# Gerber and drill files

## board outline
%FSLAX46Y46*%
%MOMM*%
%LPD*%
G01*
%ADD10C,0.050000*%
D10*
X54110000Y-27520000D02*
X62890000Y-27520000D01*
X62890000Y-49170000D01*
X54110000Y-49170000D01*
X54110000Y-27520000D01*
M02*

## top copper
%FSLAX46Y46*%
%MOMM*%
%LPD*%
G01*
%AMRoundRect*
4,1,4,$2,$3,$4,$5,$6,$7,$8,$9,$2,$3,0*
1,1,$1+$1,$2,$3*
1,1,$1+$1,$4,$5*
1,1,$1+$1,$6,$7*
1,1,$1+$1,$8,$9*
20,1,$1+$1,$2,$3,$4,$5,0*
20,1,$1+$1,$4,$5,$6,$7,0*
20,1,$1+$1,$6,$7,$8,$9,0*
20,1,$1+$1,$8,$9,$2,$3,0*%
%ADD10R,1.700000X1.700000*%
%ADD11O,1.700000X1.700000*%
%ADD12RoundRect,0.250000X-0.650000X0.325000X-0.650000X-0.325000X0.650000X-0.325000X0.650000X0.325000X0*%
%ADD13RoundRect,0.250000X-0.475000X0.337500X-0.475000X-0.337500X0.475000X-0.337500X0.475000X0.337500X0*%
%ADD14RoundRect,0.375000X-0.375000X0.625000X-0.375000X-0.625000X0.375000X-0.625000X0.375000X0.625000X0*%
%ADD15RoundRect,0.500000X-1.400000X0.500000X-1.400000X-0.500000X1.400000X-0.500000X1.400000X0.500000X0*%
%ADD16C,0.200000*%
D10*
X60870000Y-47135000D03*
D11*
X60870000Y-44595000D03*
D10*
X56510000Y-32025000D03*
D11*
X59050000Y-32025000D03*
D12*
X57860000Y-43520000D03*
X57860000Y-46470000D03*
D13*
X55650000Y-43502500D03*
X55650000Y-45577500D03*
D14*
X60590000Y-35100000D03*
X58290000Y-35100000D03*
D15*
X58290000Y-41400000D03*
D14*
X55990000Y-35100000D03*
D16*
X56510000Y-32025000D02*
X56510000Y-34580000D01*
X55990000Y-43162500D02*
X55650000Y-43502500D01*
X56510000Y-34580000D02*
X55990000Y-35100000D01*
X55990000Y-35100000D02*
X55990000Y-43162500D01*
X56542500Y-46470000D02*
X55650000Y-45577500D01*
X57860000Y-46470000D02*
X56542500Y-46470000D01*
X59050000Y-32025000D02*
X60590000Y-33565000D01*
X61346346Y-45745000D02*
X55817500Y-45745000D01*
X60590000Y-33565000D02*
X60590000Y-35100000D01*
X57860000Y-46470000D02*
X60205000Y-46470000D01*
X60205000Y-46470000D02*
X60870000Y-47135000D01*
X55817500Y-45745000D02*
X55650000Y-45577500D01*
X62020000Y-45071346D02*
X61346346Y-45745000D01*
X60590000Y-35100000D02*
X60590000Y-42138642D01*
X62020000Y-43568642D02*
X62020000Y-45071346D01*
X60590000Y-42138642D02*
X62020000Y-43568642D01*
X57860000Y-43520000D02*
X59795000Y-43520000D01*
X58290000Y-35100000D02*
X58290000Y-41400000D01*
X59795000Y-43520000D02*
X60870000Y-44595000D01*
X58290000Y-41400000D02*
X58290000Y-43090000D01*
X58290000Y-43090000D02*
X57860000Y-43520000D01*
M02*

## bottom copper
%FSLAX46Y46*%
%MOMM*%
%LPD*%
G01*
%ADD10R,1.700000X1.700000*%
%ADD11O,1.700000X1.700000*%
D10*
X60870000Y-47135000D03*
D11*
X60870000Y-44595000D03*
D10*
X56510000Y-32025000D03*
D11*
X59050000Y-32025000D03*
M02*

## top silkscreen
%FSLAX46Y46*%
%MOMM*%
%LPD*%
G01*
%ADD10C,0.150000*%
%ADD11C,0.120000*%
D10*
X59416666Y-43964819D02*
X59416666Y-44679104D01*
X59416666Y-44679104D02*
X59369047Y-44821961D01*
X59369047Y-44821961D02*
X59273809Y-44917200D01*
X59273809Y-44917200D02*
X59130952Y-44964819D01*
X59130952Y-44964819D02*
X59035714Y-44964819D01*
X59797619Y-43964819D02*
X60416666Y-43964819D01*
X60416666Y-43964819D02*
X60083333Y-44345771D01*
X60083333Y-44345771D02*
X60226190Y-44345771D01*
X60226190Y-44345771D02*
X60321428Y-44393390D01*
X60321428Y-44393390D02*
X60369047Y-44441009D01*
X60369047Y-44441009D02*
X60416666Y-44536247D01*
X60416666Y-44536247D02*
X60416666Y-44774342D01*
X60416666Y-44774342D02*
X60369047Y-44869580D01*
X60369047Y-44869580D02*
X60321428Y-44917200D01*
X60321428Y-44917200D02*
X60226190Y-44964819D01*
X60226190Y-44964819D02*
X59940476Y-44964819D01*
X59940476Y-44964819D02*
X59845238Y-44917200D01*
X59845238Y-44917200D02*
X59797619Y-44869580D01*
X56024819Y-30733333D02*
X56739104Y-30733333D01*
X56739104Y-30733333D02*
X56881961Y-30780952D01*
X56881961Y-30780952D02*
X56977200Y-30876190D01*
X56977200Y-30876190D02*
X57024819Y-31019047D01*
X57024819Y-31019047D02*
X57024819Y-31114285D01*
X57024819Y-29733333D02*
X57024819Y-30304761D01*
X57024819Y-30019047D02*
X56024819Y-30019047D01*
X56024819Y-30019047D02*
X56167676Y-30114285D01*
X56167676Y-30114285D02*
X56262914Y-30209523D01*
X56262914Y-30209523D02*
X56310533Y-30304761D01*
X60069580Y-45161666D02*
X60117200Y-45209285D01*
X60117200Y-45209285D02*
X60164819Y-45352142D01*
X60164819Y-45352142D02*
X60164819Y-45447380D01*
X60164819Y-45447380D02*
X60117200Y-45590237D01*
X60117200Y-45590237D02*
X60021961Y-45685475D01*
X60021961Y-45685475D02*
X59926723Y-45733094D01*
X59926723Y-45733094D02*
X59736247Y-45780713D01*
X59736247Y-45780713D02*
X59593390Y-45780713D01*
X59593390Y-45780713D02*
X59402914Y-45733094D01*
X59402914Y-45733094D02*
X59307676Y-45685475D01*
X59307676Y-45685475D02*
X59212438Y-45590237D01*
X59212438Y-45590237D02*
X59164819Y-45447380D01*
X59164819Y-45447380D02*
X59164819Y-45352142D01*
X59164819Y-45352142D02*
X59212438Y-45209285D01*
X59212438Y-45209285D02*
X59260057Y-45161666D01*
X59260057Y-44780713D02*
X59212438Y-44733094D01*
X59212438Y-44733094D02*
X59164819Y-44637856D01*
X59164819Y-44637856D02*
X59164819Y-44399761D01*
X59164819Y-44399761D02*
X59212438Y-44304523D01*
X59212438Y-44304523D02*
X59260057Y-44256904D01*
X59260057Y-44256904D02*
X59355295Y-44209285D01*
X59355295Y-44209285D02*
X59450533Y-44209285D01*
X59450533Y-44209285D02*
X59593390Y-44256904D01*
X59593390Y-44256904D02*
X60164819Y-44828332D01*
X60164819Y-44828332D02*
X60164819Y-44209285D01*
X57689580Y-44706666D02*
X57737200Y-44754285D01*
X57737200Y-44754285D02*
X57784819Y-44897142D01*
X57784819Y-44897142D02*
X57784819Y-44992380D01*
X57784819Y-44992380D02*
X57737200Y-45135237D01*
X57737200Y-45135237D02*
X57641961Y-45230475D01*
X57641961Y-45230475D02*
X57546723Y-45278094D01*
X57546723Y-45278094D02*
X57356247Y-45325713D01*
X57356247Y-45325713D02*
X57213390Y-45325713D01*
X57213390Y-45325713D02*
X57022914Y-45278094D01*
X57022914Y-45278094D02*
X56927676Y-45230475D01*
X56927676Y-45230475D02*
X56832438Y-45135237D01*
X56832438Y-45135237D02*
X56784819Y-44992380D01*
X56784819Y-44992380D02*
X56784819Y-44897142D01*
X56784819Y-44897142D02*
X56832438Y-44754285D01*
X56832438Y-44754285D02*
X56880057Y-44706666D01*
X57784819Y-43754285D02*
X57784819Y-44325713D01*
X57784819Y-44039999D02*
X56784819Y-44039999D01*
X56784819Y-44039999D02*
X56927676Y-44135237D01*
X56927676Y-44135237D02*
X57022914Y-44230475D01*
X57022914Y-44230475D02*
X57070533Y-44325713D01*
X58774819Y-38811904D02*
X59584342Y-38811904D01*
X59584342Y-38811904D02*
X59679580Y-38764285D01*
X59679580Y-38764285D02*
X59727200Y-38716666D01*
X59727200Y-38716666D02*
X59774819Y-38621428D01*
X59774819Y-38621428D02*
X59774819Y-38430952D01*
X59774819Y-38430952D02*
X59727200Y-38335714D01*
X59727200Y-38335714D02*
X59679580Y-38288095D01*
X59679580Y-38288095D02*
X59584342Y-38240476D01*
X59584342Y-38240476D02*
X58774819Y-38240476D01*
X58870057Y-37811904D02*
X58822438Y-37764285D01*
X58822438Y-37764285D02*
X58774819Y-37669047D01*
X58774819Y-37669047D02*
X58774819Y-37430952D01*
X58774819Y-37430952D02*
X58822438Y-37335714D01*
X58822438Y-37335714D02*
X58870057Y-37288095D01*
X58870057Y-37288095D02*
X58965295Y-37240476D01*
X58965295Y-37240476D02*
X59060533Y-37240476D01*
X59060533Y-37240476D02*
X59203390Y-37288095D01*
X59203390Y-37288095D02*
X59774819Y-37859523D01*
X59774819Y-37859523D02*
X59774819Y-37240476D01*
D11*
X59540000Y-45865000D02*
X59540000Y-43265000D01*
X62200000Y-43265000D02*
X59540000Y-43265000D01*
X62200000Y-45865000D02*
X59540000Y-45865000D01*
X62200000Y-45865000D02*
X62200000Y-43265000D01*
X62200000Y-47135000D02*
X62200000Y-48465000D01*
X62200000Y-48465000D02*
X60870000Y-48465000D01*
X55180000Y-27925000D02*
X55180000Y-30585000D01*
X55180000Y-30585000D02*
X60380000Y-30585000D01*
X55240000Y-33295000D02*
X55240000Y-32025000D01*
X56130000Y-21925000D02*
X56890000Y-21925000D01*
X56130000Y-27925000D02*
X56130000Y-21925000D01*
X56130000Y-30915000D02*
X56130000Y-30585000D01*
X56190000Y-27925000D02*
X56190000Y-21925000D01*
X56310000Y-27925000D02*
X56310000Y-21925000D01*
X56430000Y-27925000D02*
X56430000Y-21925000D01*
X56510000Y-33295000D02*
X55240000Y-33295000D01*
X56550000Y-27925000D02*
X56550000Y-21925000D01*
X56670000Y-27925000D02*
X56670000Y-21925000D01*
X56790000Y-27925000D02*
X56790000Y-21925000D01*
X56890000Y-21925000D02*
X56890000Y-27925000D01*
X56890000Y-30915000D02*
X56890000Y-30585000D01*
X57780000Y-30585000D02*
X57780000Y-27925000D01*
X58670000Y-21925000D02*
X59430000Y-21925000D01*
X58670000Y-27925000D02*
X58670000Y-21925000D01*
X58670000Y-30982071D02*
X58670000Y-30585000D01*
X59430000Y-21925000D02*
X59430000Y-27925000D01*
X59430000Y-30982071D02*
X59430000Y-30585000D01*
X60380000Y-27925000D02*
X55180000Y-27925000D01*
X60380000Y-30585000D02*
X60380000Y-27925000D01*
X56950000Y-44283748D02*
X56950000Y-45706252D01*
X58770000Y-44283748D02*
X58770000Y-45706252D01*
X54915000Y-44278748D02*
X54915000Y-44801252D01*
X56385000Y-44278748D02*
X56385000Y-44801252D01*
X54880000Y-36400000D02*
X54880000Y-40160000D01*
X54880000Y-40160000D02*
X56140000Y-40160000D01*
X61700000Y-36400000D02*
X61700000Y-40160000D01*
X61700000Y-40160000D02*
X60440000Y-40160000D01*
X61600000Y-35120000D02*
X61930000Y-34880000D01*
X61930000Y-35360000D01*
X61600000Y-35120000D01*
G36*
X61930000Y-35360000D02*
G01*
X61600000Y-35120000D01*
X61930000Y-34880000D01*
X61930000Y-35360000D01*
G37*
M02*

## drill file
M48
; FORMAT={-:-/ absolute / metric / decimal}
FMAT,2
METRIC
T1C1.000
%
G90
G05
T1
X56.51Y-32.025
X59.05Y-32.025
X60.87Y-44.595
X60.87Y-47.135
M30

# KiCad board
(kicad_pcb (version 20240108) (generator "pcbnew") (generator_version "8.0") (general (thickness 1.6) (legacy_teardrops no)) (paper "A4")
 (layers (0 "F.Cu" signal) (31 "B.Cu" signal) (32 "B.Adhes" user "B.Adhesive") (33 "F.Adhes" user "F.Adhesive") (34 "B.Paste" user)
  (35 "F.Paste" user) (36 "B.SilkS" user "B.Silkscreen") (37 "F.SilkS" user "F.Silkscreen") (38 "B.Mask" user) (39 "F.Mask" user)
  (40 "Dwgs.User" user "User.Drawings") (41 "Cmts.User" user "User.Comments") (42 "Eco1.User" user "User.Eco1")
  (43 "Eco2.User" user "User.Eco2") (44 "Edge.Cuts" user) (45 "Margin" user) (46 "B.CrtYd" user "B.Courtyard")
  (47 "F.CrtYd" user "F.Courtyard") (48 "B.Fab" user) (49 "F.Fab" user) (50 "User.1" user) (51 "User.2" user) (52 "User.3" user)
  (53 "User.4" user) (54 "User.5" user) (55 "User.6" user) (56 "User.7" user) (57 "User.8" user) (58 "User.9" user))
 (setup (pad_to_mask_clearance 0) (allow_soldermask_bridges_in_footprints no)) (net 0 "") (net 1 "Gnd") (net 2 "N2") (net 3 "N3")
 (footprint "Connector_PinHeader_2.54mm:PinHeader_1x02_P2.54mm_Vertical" (layer "F.Cu") (at 60.87 47.135 180)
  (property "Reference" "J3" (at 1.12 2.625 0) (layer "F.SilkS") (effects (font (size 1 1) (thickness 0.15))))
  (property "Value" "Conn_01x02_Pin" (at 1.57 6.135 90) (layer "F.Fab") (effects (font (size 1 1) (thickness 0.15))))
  (fp_line (start 1.33 1.27) (end 1.33 3.87) (stroke (width 0.12) (type solid)) (layer "F.SilkS"))
  (fp_line (start -1.33 3.87) (end 1.33 3.87) (stroke (width 0.12) (type solid)) (layer "F.SilkS"))
  (fp_line (start -1.33 1.27) (end 1.33 1.27) (stroke (width 0.12) (type solid)) (layer "F.SilkS"))
  (fp_line (start -1.33 1.27) (end -1.33 3.87) (stroke (width 0.12) (type solid)) (layer "F.SilkS"))
  (fp_line (start -1.33 0) (end -1.33 -1.33) (stroke (width 0.12) (type solid)) (layer "F.SilkS"))
  (fp_line (start -1.33 -1.33) (end 0 -1.33) (stroke (width 0.12) (type solid)) (layer "F.SilkS"))
  (pad "1" thru_hole rect (at 0 0 180) (size 1.7 1.7) (drill 1) (layers "*.Cu" "*.Mask") (remove_unused_layers no) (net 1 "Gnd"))
  (pad "2" thru_hole oval (at 0 2.54 180) (size 1.7 1.7) (drill 1) (layers "*.Cu" "*.Mask") (remove_unused_layers no) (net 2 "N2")))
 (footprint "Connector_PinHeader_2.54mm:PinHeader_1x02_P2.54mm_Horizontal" (layer "F.Cu") (at 56.51 32.025 90)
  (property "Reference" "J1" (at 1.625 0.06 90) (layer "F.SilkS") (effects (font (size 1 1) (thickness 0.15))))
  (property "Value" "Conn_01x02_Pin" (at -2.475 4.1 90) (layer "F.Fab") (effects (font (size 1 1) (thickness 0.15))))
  (fp_line (start 4.1 -1.33) (end 1.44 -1.33) (stroke (width 0.12) (type solid)) (layer "F.SilkS"))
  (fp_line (start 1.44 -1.33) (end 1.44 3.87) (stroke (width 0.12) (type solid)) (layer "F.SilkS"))
  (fp_line (start -1.27 -1.27) (end 0 -1.27) (stroke (width 0.12) (type solid)) (layer "F.SilkS"))
  (fp_line (start 10.1 -0.38) (end 10.1 0.38) (stroke (width 0.12) (type solid)) (layer "F.SilkS"))
  (fp_line (start 4.1 -0.38) (end 10.1 -0.38) (stroke (width 0.12) (type solid)) (layer "F.SilkS"))
  (fp_line (start 1.11 -0.38) (end 1.44 -0.38) (stroke (width 0.12) (type solid)) (layer "F.SilkS"))
  (fp_line (start 4.1 -0.32) (end 10.1 -0.32) (stroke (width 0.12) (type solid)) (layer "F.SilkS"))
  (fp_line (start 4.1 -0.2) (end 10.1 -0.2) (stroke (width 0.12) (type solid)) (layer "F.SilkS"))
  (fp_line (start 4.1 -0.08) (end 10.1 -0.08) (stroke (width 0.12) (type solid)) (layer "F.SilkS"))
  (fp_line (start -1.27 0) (end -1.27 -1.27) (stroke (width 0.12) (type solid)) (layer "F.SilkS"))
  (fp_line (start 4.1 0.04) (end 10.1 0.04) (stroke (width 0.12) (type solid)) (layer "F.SilkS"))
  (fp_line (start 4.1 0.16) (end 10.1 0.16) (stroke (width 0.12) (type solid)) (layer "F.SilkS"))
  (fp_line (start 4.1 0.28) (end 10.1 0.28) (stroke (width 0.12) (type solid)) (layer "F.SilkS"))
  (fp_line (start 10.1 0.38) (end 4.1 0.38) (stroke (width 0.12) (type solid)) (layer "F.SilkS"))
  (fp_line (start 1.11 0.38) (end 1.44 0.38) (stroke (width 0.12) (type solid)) (layer "F.SilkS"))
  (fp_line (start 1.44 1.27) (end 4.1 1.27) (stroke (width 0.12) (type solid)) (layer "F.SilkS"))
  (fp_line (start 10.1 2.16) (end 10.1 2.92) (stroke (width 0.12) (type solid)) (layer "F.SilkS"))
  (fp_line (start 4.1 2.16) (end 10.1 2.16) (stroke (width 0.12) (type solid)) (layer "F.SilkS"))
  (fp_line (start 1.042929 2.16) (end 1.44 2.16) (stroke (width 0.12) (type solid)) (layer "F.SilkS"))
  (fp_line (start 10.1 2.92) (end 4.1 2.92) (stroke (width 0.12) (type solid)) (layer "F.SilkS"))
  (fp_line (start 1.042929 2.92) (end 1.44 2.92) (stroke (width 0.12) (type solid)) (layer "F.SilkS"))
  (fp_line (start 4.1 3.87) (end 4.1 -1.33) (stroke (width 0.12) (type solid)) (layer "F.SilkS"))
  (fp_line (start 1.44 3.87) (end 4.1 3.87) (stroke (width 0.12) (type solid)) (layer "F.SilkS"))
  (pad "1" thru_hole rect (at 0 0 90) (size 1.7 1.7) (drill 1) (layers "*.Cu" "*.Mask") (remove_unused_layers no) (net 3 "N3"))
  (pad "2" thru_hole oval (at 0 2.54 90) (size 1.7 1.7) (drill 1) (layers "*.Cu" "*.Mask") (remove_unused_layers no) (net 1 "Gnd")))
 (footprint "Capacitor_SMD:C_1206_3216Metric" (layer "F.Cu") (at 57.86 44.995 -90)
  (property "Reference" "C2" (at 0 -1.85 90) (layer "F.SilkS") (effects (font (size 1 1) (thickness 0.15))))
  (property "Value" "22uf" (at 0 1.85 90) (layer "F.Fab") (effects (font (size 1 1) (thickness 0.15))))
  (fp_line (start -0.711252 0.91) (end 0.711252 0.91) (stroke (width 0.12) (type solid)) (layer "F.SilkS"))
  (fp_line (start -0.711252 -0.91) (end 0.711252 -0.91) (stroke (width 0.12) (type solid)) (layer "F.SilkS"))
  (pad "1" smd roundrect (at -1.475 0 270) (size 1.15 1.8) (layers "F.Cu" "F.Paste" "F.Mask") (roundrect_rratio 0.217391) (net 2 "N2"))
  (pad "2" smd roundrect (at 1.475 0 270) (size 1.15 1.8) (layers "F.Cu" "F.Paste" "F.Mask") (roundrect_rratio 0.217391) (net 1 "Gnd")))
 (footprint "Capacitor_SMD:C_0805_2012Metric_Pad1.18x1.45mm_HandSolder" (layer "F.Cu") (at 55.65 44.54 -90)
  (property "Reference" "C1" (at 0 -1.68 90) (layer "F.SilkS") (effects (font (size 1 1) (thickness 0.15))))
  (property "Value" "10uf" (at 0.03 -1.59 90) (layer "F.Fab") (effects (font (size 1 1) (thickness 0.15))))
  (fp_line (start -0.261252 0.735) (end 0.261252 0.735) (stroke (width 0.12) (type solid)) (layer "F.SilkS"))
  (fp_line (start -0.261252 -0.735) (end 0.261252 -0.735) (stroke (width 0.12) (type solid)) (layer "F.SilkS"))
  (pad "1" smd roundrect (at -1.0375 0 270) (size 1.175 1.45) (layers "F.Cu" "F.Paste" "F.Mask") (roundrect_rratio 0.212766) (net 3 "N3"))
  (pad "2" smd roundrect (at 1.0375 0 270) (size 1.175 1.45) (layers "F.Cu" "F.Paste" "F.Mask") (roundrect_rratio 0.212766) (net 1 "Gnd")))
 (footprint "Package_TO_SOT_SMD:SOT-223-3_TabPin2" (layer "F.Cu") (at 58.29 38.25 -90)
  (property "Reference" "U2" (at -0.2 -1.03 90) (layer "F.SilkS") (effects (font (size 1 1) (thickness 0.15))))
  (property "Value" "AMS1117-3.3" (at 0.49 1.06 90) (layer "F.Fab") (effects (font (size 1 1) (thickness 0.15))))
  (fp_line (start -1.85 3.41) (end 1.91 3.41) (stroke (width 0.12) (type solid)) (layer "F.SilkS"))
  (fp_line (start 1.91 3.41) (end 1.91 2.15) (stroke (width 0.12) (type solid)) (layer "F.SilkS"))
  (fp_line (start -1.85 -3.41) (end 1.91 -3.41) (stroke (width 0.12) (type solid)) (layer "F.SilkS"))
  (fp_line (start 1.91 -3.41) (end 1.91 -2.15) (stroke (width 0.12) (type solid)) (layer "F.SilkS"))
  (fp_poly
   (pts (xy -3.13 -3.31) (xy -3.37 -3.64) (xy -2.89 -3.64) (xy -3.13 -3.31)) (stroke (width 0.12) (type solid)) (fill solid)
   (layer "F.SilkS"))
  (pad "1" smd roundrect (at -3.15 -2.3 270) (size 2 1.5) (layers "F.Cu" "F.Paste" "F.Mask") (roundrect_rratio 0.25) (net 1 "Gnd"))
  (pad "2" smd roundrect (at -3.15 0 270) (size 2 1.5) (layers "F.Cu" "F.Paste" "F.Mask") (roundrect_rratio 0.25) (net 2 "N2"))
  (pad "2" smd roundrect (at 3.15 0 270) (size 2 3.8) (layers "F.Cu" "F.Paste" "F.Mask") (roundrect_rratio 0.25) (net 2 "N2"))
  (pad "3" smd roundrect (at -3.15 2.3 270) (size 2 1.5) (layers "F.Cu" "F.Paste" "F.Mask") (roundrect_rratio 0.25) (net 3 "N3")))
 (gr_rect (start 54.11 27.52) (end 62.89 49.17) (stroke (width 0.05) (type default)) (fill none) (layer "Edge.Cuts"))
 (segment (start 56.51 32.025) (end 56.51 34.58) (width 0.2) (layer "F.Cu") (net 3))
 (segment (start 55.99 43.1625) (end 55.65 43.5025) (width 0.2) (layer "F.Cu") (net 3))
 (segment (start 56.51 34.58) (end 55.99 35.1) (width 0.2) (layer "F.Cu") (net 3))
 (segment (start 55.99 35.1) (end 55.99 43.1625) (width 0.2) (layer "F.Cu") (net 3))
 (segment (start 56.5425 46.47) (end 55.65 45.5775) (width 0.2) (layer "F.Cu") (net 1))
 (segment (start 57.86 46.47) (end 56.5425 46.47) (width 0.2) (layer "F.Cu") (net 1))
 (segment (start 59.05 32.025) (end 60.59 33.565) (width 0.2) (layer "F.Cu") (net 1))
 (segment (start 61.346346 45.745) (end 55.8175 45.745) (width 0.2) (layer "F.Cu") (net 1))
 (segment (start 60.59 33.565) (end 60.59 35.1) (width 0.2) (layer "F.Cu") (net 1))
 (segment (start 57.86 46.47) (end 60.205 46.47) (width 0.2) (layer "F.Cu") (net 1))
 (segment (start 60.205 46.47) (end 60.87 47.135) (width 0.2) (layer "F.Cu") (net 1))
 (segment (start 55.8175 45.745) (end 55.65 45.5775) (width 0.2) (layer "F.Cu") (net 1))
 (segment (start 62.02 45.071346) (end 61.346346 45.745) (width 0.2) (layer "F.Cu") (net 1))
 (segment (start 60.59 35.1) (end 60.59 42.138642) (width 0.2) (layer "F.Cu") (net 1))
 (segment (start 62.02 43.568642) (end 62.02 45.071346) (width 0.2) (layer "F.Cu") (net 1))
 (segment (start 60.59 42.138642) (end 62.02 43.568642) (width 0.2) (layer "F.Cu") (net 1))
 (segment (start 57.86 43.52) (end 59.795 43.52) (width 0.2) (layer "F.Cu") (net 2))
 (segment (start 58.29 35.1) (end 58.29 41.4) (width 0.2) (layer "F.Cu") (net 2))
 (segment (start 59.795 43.52) (end 60.87 44.595) (width 0.2) (layer "F.Cu") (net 2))
 (segment (start 58.29 41.4) (end 58.29 43.09) (width 0.2) (layer "F.Cu") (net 2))
 (segment (start 58.29 43.09) (end 57.86 43.52) (width 0.2) (layer "F.Cu") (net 2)))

